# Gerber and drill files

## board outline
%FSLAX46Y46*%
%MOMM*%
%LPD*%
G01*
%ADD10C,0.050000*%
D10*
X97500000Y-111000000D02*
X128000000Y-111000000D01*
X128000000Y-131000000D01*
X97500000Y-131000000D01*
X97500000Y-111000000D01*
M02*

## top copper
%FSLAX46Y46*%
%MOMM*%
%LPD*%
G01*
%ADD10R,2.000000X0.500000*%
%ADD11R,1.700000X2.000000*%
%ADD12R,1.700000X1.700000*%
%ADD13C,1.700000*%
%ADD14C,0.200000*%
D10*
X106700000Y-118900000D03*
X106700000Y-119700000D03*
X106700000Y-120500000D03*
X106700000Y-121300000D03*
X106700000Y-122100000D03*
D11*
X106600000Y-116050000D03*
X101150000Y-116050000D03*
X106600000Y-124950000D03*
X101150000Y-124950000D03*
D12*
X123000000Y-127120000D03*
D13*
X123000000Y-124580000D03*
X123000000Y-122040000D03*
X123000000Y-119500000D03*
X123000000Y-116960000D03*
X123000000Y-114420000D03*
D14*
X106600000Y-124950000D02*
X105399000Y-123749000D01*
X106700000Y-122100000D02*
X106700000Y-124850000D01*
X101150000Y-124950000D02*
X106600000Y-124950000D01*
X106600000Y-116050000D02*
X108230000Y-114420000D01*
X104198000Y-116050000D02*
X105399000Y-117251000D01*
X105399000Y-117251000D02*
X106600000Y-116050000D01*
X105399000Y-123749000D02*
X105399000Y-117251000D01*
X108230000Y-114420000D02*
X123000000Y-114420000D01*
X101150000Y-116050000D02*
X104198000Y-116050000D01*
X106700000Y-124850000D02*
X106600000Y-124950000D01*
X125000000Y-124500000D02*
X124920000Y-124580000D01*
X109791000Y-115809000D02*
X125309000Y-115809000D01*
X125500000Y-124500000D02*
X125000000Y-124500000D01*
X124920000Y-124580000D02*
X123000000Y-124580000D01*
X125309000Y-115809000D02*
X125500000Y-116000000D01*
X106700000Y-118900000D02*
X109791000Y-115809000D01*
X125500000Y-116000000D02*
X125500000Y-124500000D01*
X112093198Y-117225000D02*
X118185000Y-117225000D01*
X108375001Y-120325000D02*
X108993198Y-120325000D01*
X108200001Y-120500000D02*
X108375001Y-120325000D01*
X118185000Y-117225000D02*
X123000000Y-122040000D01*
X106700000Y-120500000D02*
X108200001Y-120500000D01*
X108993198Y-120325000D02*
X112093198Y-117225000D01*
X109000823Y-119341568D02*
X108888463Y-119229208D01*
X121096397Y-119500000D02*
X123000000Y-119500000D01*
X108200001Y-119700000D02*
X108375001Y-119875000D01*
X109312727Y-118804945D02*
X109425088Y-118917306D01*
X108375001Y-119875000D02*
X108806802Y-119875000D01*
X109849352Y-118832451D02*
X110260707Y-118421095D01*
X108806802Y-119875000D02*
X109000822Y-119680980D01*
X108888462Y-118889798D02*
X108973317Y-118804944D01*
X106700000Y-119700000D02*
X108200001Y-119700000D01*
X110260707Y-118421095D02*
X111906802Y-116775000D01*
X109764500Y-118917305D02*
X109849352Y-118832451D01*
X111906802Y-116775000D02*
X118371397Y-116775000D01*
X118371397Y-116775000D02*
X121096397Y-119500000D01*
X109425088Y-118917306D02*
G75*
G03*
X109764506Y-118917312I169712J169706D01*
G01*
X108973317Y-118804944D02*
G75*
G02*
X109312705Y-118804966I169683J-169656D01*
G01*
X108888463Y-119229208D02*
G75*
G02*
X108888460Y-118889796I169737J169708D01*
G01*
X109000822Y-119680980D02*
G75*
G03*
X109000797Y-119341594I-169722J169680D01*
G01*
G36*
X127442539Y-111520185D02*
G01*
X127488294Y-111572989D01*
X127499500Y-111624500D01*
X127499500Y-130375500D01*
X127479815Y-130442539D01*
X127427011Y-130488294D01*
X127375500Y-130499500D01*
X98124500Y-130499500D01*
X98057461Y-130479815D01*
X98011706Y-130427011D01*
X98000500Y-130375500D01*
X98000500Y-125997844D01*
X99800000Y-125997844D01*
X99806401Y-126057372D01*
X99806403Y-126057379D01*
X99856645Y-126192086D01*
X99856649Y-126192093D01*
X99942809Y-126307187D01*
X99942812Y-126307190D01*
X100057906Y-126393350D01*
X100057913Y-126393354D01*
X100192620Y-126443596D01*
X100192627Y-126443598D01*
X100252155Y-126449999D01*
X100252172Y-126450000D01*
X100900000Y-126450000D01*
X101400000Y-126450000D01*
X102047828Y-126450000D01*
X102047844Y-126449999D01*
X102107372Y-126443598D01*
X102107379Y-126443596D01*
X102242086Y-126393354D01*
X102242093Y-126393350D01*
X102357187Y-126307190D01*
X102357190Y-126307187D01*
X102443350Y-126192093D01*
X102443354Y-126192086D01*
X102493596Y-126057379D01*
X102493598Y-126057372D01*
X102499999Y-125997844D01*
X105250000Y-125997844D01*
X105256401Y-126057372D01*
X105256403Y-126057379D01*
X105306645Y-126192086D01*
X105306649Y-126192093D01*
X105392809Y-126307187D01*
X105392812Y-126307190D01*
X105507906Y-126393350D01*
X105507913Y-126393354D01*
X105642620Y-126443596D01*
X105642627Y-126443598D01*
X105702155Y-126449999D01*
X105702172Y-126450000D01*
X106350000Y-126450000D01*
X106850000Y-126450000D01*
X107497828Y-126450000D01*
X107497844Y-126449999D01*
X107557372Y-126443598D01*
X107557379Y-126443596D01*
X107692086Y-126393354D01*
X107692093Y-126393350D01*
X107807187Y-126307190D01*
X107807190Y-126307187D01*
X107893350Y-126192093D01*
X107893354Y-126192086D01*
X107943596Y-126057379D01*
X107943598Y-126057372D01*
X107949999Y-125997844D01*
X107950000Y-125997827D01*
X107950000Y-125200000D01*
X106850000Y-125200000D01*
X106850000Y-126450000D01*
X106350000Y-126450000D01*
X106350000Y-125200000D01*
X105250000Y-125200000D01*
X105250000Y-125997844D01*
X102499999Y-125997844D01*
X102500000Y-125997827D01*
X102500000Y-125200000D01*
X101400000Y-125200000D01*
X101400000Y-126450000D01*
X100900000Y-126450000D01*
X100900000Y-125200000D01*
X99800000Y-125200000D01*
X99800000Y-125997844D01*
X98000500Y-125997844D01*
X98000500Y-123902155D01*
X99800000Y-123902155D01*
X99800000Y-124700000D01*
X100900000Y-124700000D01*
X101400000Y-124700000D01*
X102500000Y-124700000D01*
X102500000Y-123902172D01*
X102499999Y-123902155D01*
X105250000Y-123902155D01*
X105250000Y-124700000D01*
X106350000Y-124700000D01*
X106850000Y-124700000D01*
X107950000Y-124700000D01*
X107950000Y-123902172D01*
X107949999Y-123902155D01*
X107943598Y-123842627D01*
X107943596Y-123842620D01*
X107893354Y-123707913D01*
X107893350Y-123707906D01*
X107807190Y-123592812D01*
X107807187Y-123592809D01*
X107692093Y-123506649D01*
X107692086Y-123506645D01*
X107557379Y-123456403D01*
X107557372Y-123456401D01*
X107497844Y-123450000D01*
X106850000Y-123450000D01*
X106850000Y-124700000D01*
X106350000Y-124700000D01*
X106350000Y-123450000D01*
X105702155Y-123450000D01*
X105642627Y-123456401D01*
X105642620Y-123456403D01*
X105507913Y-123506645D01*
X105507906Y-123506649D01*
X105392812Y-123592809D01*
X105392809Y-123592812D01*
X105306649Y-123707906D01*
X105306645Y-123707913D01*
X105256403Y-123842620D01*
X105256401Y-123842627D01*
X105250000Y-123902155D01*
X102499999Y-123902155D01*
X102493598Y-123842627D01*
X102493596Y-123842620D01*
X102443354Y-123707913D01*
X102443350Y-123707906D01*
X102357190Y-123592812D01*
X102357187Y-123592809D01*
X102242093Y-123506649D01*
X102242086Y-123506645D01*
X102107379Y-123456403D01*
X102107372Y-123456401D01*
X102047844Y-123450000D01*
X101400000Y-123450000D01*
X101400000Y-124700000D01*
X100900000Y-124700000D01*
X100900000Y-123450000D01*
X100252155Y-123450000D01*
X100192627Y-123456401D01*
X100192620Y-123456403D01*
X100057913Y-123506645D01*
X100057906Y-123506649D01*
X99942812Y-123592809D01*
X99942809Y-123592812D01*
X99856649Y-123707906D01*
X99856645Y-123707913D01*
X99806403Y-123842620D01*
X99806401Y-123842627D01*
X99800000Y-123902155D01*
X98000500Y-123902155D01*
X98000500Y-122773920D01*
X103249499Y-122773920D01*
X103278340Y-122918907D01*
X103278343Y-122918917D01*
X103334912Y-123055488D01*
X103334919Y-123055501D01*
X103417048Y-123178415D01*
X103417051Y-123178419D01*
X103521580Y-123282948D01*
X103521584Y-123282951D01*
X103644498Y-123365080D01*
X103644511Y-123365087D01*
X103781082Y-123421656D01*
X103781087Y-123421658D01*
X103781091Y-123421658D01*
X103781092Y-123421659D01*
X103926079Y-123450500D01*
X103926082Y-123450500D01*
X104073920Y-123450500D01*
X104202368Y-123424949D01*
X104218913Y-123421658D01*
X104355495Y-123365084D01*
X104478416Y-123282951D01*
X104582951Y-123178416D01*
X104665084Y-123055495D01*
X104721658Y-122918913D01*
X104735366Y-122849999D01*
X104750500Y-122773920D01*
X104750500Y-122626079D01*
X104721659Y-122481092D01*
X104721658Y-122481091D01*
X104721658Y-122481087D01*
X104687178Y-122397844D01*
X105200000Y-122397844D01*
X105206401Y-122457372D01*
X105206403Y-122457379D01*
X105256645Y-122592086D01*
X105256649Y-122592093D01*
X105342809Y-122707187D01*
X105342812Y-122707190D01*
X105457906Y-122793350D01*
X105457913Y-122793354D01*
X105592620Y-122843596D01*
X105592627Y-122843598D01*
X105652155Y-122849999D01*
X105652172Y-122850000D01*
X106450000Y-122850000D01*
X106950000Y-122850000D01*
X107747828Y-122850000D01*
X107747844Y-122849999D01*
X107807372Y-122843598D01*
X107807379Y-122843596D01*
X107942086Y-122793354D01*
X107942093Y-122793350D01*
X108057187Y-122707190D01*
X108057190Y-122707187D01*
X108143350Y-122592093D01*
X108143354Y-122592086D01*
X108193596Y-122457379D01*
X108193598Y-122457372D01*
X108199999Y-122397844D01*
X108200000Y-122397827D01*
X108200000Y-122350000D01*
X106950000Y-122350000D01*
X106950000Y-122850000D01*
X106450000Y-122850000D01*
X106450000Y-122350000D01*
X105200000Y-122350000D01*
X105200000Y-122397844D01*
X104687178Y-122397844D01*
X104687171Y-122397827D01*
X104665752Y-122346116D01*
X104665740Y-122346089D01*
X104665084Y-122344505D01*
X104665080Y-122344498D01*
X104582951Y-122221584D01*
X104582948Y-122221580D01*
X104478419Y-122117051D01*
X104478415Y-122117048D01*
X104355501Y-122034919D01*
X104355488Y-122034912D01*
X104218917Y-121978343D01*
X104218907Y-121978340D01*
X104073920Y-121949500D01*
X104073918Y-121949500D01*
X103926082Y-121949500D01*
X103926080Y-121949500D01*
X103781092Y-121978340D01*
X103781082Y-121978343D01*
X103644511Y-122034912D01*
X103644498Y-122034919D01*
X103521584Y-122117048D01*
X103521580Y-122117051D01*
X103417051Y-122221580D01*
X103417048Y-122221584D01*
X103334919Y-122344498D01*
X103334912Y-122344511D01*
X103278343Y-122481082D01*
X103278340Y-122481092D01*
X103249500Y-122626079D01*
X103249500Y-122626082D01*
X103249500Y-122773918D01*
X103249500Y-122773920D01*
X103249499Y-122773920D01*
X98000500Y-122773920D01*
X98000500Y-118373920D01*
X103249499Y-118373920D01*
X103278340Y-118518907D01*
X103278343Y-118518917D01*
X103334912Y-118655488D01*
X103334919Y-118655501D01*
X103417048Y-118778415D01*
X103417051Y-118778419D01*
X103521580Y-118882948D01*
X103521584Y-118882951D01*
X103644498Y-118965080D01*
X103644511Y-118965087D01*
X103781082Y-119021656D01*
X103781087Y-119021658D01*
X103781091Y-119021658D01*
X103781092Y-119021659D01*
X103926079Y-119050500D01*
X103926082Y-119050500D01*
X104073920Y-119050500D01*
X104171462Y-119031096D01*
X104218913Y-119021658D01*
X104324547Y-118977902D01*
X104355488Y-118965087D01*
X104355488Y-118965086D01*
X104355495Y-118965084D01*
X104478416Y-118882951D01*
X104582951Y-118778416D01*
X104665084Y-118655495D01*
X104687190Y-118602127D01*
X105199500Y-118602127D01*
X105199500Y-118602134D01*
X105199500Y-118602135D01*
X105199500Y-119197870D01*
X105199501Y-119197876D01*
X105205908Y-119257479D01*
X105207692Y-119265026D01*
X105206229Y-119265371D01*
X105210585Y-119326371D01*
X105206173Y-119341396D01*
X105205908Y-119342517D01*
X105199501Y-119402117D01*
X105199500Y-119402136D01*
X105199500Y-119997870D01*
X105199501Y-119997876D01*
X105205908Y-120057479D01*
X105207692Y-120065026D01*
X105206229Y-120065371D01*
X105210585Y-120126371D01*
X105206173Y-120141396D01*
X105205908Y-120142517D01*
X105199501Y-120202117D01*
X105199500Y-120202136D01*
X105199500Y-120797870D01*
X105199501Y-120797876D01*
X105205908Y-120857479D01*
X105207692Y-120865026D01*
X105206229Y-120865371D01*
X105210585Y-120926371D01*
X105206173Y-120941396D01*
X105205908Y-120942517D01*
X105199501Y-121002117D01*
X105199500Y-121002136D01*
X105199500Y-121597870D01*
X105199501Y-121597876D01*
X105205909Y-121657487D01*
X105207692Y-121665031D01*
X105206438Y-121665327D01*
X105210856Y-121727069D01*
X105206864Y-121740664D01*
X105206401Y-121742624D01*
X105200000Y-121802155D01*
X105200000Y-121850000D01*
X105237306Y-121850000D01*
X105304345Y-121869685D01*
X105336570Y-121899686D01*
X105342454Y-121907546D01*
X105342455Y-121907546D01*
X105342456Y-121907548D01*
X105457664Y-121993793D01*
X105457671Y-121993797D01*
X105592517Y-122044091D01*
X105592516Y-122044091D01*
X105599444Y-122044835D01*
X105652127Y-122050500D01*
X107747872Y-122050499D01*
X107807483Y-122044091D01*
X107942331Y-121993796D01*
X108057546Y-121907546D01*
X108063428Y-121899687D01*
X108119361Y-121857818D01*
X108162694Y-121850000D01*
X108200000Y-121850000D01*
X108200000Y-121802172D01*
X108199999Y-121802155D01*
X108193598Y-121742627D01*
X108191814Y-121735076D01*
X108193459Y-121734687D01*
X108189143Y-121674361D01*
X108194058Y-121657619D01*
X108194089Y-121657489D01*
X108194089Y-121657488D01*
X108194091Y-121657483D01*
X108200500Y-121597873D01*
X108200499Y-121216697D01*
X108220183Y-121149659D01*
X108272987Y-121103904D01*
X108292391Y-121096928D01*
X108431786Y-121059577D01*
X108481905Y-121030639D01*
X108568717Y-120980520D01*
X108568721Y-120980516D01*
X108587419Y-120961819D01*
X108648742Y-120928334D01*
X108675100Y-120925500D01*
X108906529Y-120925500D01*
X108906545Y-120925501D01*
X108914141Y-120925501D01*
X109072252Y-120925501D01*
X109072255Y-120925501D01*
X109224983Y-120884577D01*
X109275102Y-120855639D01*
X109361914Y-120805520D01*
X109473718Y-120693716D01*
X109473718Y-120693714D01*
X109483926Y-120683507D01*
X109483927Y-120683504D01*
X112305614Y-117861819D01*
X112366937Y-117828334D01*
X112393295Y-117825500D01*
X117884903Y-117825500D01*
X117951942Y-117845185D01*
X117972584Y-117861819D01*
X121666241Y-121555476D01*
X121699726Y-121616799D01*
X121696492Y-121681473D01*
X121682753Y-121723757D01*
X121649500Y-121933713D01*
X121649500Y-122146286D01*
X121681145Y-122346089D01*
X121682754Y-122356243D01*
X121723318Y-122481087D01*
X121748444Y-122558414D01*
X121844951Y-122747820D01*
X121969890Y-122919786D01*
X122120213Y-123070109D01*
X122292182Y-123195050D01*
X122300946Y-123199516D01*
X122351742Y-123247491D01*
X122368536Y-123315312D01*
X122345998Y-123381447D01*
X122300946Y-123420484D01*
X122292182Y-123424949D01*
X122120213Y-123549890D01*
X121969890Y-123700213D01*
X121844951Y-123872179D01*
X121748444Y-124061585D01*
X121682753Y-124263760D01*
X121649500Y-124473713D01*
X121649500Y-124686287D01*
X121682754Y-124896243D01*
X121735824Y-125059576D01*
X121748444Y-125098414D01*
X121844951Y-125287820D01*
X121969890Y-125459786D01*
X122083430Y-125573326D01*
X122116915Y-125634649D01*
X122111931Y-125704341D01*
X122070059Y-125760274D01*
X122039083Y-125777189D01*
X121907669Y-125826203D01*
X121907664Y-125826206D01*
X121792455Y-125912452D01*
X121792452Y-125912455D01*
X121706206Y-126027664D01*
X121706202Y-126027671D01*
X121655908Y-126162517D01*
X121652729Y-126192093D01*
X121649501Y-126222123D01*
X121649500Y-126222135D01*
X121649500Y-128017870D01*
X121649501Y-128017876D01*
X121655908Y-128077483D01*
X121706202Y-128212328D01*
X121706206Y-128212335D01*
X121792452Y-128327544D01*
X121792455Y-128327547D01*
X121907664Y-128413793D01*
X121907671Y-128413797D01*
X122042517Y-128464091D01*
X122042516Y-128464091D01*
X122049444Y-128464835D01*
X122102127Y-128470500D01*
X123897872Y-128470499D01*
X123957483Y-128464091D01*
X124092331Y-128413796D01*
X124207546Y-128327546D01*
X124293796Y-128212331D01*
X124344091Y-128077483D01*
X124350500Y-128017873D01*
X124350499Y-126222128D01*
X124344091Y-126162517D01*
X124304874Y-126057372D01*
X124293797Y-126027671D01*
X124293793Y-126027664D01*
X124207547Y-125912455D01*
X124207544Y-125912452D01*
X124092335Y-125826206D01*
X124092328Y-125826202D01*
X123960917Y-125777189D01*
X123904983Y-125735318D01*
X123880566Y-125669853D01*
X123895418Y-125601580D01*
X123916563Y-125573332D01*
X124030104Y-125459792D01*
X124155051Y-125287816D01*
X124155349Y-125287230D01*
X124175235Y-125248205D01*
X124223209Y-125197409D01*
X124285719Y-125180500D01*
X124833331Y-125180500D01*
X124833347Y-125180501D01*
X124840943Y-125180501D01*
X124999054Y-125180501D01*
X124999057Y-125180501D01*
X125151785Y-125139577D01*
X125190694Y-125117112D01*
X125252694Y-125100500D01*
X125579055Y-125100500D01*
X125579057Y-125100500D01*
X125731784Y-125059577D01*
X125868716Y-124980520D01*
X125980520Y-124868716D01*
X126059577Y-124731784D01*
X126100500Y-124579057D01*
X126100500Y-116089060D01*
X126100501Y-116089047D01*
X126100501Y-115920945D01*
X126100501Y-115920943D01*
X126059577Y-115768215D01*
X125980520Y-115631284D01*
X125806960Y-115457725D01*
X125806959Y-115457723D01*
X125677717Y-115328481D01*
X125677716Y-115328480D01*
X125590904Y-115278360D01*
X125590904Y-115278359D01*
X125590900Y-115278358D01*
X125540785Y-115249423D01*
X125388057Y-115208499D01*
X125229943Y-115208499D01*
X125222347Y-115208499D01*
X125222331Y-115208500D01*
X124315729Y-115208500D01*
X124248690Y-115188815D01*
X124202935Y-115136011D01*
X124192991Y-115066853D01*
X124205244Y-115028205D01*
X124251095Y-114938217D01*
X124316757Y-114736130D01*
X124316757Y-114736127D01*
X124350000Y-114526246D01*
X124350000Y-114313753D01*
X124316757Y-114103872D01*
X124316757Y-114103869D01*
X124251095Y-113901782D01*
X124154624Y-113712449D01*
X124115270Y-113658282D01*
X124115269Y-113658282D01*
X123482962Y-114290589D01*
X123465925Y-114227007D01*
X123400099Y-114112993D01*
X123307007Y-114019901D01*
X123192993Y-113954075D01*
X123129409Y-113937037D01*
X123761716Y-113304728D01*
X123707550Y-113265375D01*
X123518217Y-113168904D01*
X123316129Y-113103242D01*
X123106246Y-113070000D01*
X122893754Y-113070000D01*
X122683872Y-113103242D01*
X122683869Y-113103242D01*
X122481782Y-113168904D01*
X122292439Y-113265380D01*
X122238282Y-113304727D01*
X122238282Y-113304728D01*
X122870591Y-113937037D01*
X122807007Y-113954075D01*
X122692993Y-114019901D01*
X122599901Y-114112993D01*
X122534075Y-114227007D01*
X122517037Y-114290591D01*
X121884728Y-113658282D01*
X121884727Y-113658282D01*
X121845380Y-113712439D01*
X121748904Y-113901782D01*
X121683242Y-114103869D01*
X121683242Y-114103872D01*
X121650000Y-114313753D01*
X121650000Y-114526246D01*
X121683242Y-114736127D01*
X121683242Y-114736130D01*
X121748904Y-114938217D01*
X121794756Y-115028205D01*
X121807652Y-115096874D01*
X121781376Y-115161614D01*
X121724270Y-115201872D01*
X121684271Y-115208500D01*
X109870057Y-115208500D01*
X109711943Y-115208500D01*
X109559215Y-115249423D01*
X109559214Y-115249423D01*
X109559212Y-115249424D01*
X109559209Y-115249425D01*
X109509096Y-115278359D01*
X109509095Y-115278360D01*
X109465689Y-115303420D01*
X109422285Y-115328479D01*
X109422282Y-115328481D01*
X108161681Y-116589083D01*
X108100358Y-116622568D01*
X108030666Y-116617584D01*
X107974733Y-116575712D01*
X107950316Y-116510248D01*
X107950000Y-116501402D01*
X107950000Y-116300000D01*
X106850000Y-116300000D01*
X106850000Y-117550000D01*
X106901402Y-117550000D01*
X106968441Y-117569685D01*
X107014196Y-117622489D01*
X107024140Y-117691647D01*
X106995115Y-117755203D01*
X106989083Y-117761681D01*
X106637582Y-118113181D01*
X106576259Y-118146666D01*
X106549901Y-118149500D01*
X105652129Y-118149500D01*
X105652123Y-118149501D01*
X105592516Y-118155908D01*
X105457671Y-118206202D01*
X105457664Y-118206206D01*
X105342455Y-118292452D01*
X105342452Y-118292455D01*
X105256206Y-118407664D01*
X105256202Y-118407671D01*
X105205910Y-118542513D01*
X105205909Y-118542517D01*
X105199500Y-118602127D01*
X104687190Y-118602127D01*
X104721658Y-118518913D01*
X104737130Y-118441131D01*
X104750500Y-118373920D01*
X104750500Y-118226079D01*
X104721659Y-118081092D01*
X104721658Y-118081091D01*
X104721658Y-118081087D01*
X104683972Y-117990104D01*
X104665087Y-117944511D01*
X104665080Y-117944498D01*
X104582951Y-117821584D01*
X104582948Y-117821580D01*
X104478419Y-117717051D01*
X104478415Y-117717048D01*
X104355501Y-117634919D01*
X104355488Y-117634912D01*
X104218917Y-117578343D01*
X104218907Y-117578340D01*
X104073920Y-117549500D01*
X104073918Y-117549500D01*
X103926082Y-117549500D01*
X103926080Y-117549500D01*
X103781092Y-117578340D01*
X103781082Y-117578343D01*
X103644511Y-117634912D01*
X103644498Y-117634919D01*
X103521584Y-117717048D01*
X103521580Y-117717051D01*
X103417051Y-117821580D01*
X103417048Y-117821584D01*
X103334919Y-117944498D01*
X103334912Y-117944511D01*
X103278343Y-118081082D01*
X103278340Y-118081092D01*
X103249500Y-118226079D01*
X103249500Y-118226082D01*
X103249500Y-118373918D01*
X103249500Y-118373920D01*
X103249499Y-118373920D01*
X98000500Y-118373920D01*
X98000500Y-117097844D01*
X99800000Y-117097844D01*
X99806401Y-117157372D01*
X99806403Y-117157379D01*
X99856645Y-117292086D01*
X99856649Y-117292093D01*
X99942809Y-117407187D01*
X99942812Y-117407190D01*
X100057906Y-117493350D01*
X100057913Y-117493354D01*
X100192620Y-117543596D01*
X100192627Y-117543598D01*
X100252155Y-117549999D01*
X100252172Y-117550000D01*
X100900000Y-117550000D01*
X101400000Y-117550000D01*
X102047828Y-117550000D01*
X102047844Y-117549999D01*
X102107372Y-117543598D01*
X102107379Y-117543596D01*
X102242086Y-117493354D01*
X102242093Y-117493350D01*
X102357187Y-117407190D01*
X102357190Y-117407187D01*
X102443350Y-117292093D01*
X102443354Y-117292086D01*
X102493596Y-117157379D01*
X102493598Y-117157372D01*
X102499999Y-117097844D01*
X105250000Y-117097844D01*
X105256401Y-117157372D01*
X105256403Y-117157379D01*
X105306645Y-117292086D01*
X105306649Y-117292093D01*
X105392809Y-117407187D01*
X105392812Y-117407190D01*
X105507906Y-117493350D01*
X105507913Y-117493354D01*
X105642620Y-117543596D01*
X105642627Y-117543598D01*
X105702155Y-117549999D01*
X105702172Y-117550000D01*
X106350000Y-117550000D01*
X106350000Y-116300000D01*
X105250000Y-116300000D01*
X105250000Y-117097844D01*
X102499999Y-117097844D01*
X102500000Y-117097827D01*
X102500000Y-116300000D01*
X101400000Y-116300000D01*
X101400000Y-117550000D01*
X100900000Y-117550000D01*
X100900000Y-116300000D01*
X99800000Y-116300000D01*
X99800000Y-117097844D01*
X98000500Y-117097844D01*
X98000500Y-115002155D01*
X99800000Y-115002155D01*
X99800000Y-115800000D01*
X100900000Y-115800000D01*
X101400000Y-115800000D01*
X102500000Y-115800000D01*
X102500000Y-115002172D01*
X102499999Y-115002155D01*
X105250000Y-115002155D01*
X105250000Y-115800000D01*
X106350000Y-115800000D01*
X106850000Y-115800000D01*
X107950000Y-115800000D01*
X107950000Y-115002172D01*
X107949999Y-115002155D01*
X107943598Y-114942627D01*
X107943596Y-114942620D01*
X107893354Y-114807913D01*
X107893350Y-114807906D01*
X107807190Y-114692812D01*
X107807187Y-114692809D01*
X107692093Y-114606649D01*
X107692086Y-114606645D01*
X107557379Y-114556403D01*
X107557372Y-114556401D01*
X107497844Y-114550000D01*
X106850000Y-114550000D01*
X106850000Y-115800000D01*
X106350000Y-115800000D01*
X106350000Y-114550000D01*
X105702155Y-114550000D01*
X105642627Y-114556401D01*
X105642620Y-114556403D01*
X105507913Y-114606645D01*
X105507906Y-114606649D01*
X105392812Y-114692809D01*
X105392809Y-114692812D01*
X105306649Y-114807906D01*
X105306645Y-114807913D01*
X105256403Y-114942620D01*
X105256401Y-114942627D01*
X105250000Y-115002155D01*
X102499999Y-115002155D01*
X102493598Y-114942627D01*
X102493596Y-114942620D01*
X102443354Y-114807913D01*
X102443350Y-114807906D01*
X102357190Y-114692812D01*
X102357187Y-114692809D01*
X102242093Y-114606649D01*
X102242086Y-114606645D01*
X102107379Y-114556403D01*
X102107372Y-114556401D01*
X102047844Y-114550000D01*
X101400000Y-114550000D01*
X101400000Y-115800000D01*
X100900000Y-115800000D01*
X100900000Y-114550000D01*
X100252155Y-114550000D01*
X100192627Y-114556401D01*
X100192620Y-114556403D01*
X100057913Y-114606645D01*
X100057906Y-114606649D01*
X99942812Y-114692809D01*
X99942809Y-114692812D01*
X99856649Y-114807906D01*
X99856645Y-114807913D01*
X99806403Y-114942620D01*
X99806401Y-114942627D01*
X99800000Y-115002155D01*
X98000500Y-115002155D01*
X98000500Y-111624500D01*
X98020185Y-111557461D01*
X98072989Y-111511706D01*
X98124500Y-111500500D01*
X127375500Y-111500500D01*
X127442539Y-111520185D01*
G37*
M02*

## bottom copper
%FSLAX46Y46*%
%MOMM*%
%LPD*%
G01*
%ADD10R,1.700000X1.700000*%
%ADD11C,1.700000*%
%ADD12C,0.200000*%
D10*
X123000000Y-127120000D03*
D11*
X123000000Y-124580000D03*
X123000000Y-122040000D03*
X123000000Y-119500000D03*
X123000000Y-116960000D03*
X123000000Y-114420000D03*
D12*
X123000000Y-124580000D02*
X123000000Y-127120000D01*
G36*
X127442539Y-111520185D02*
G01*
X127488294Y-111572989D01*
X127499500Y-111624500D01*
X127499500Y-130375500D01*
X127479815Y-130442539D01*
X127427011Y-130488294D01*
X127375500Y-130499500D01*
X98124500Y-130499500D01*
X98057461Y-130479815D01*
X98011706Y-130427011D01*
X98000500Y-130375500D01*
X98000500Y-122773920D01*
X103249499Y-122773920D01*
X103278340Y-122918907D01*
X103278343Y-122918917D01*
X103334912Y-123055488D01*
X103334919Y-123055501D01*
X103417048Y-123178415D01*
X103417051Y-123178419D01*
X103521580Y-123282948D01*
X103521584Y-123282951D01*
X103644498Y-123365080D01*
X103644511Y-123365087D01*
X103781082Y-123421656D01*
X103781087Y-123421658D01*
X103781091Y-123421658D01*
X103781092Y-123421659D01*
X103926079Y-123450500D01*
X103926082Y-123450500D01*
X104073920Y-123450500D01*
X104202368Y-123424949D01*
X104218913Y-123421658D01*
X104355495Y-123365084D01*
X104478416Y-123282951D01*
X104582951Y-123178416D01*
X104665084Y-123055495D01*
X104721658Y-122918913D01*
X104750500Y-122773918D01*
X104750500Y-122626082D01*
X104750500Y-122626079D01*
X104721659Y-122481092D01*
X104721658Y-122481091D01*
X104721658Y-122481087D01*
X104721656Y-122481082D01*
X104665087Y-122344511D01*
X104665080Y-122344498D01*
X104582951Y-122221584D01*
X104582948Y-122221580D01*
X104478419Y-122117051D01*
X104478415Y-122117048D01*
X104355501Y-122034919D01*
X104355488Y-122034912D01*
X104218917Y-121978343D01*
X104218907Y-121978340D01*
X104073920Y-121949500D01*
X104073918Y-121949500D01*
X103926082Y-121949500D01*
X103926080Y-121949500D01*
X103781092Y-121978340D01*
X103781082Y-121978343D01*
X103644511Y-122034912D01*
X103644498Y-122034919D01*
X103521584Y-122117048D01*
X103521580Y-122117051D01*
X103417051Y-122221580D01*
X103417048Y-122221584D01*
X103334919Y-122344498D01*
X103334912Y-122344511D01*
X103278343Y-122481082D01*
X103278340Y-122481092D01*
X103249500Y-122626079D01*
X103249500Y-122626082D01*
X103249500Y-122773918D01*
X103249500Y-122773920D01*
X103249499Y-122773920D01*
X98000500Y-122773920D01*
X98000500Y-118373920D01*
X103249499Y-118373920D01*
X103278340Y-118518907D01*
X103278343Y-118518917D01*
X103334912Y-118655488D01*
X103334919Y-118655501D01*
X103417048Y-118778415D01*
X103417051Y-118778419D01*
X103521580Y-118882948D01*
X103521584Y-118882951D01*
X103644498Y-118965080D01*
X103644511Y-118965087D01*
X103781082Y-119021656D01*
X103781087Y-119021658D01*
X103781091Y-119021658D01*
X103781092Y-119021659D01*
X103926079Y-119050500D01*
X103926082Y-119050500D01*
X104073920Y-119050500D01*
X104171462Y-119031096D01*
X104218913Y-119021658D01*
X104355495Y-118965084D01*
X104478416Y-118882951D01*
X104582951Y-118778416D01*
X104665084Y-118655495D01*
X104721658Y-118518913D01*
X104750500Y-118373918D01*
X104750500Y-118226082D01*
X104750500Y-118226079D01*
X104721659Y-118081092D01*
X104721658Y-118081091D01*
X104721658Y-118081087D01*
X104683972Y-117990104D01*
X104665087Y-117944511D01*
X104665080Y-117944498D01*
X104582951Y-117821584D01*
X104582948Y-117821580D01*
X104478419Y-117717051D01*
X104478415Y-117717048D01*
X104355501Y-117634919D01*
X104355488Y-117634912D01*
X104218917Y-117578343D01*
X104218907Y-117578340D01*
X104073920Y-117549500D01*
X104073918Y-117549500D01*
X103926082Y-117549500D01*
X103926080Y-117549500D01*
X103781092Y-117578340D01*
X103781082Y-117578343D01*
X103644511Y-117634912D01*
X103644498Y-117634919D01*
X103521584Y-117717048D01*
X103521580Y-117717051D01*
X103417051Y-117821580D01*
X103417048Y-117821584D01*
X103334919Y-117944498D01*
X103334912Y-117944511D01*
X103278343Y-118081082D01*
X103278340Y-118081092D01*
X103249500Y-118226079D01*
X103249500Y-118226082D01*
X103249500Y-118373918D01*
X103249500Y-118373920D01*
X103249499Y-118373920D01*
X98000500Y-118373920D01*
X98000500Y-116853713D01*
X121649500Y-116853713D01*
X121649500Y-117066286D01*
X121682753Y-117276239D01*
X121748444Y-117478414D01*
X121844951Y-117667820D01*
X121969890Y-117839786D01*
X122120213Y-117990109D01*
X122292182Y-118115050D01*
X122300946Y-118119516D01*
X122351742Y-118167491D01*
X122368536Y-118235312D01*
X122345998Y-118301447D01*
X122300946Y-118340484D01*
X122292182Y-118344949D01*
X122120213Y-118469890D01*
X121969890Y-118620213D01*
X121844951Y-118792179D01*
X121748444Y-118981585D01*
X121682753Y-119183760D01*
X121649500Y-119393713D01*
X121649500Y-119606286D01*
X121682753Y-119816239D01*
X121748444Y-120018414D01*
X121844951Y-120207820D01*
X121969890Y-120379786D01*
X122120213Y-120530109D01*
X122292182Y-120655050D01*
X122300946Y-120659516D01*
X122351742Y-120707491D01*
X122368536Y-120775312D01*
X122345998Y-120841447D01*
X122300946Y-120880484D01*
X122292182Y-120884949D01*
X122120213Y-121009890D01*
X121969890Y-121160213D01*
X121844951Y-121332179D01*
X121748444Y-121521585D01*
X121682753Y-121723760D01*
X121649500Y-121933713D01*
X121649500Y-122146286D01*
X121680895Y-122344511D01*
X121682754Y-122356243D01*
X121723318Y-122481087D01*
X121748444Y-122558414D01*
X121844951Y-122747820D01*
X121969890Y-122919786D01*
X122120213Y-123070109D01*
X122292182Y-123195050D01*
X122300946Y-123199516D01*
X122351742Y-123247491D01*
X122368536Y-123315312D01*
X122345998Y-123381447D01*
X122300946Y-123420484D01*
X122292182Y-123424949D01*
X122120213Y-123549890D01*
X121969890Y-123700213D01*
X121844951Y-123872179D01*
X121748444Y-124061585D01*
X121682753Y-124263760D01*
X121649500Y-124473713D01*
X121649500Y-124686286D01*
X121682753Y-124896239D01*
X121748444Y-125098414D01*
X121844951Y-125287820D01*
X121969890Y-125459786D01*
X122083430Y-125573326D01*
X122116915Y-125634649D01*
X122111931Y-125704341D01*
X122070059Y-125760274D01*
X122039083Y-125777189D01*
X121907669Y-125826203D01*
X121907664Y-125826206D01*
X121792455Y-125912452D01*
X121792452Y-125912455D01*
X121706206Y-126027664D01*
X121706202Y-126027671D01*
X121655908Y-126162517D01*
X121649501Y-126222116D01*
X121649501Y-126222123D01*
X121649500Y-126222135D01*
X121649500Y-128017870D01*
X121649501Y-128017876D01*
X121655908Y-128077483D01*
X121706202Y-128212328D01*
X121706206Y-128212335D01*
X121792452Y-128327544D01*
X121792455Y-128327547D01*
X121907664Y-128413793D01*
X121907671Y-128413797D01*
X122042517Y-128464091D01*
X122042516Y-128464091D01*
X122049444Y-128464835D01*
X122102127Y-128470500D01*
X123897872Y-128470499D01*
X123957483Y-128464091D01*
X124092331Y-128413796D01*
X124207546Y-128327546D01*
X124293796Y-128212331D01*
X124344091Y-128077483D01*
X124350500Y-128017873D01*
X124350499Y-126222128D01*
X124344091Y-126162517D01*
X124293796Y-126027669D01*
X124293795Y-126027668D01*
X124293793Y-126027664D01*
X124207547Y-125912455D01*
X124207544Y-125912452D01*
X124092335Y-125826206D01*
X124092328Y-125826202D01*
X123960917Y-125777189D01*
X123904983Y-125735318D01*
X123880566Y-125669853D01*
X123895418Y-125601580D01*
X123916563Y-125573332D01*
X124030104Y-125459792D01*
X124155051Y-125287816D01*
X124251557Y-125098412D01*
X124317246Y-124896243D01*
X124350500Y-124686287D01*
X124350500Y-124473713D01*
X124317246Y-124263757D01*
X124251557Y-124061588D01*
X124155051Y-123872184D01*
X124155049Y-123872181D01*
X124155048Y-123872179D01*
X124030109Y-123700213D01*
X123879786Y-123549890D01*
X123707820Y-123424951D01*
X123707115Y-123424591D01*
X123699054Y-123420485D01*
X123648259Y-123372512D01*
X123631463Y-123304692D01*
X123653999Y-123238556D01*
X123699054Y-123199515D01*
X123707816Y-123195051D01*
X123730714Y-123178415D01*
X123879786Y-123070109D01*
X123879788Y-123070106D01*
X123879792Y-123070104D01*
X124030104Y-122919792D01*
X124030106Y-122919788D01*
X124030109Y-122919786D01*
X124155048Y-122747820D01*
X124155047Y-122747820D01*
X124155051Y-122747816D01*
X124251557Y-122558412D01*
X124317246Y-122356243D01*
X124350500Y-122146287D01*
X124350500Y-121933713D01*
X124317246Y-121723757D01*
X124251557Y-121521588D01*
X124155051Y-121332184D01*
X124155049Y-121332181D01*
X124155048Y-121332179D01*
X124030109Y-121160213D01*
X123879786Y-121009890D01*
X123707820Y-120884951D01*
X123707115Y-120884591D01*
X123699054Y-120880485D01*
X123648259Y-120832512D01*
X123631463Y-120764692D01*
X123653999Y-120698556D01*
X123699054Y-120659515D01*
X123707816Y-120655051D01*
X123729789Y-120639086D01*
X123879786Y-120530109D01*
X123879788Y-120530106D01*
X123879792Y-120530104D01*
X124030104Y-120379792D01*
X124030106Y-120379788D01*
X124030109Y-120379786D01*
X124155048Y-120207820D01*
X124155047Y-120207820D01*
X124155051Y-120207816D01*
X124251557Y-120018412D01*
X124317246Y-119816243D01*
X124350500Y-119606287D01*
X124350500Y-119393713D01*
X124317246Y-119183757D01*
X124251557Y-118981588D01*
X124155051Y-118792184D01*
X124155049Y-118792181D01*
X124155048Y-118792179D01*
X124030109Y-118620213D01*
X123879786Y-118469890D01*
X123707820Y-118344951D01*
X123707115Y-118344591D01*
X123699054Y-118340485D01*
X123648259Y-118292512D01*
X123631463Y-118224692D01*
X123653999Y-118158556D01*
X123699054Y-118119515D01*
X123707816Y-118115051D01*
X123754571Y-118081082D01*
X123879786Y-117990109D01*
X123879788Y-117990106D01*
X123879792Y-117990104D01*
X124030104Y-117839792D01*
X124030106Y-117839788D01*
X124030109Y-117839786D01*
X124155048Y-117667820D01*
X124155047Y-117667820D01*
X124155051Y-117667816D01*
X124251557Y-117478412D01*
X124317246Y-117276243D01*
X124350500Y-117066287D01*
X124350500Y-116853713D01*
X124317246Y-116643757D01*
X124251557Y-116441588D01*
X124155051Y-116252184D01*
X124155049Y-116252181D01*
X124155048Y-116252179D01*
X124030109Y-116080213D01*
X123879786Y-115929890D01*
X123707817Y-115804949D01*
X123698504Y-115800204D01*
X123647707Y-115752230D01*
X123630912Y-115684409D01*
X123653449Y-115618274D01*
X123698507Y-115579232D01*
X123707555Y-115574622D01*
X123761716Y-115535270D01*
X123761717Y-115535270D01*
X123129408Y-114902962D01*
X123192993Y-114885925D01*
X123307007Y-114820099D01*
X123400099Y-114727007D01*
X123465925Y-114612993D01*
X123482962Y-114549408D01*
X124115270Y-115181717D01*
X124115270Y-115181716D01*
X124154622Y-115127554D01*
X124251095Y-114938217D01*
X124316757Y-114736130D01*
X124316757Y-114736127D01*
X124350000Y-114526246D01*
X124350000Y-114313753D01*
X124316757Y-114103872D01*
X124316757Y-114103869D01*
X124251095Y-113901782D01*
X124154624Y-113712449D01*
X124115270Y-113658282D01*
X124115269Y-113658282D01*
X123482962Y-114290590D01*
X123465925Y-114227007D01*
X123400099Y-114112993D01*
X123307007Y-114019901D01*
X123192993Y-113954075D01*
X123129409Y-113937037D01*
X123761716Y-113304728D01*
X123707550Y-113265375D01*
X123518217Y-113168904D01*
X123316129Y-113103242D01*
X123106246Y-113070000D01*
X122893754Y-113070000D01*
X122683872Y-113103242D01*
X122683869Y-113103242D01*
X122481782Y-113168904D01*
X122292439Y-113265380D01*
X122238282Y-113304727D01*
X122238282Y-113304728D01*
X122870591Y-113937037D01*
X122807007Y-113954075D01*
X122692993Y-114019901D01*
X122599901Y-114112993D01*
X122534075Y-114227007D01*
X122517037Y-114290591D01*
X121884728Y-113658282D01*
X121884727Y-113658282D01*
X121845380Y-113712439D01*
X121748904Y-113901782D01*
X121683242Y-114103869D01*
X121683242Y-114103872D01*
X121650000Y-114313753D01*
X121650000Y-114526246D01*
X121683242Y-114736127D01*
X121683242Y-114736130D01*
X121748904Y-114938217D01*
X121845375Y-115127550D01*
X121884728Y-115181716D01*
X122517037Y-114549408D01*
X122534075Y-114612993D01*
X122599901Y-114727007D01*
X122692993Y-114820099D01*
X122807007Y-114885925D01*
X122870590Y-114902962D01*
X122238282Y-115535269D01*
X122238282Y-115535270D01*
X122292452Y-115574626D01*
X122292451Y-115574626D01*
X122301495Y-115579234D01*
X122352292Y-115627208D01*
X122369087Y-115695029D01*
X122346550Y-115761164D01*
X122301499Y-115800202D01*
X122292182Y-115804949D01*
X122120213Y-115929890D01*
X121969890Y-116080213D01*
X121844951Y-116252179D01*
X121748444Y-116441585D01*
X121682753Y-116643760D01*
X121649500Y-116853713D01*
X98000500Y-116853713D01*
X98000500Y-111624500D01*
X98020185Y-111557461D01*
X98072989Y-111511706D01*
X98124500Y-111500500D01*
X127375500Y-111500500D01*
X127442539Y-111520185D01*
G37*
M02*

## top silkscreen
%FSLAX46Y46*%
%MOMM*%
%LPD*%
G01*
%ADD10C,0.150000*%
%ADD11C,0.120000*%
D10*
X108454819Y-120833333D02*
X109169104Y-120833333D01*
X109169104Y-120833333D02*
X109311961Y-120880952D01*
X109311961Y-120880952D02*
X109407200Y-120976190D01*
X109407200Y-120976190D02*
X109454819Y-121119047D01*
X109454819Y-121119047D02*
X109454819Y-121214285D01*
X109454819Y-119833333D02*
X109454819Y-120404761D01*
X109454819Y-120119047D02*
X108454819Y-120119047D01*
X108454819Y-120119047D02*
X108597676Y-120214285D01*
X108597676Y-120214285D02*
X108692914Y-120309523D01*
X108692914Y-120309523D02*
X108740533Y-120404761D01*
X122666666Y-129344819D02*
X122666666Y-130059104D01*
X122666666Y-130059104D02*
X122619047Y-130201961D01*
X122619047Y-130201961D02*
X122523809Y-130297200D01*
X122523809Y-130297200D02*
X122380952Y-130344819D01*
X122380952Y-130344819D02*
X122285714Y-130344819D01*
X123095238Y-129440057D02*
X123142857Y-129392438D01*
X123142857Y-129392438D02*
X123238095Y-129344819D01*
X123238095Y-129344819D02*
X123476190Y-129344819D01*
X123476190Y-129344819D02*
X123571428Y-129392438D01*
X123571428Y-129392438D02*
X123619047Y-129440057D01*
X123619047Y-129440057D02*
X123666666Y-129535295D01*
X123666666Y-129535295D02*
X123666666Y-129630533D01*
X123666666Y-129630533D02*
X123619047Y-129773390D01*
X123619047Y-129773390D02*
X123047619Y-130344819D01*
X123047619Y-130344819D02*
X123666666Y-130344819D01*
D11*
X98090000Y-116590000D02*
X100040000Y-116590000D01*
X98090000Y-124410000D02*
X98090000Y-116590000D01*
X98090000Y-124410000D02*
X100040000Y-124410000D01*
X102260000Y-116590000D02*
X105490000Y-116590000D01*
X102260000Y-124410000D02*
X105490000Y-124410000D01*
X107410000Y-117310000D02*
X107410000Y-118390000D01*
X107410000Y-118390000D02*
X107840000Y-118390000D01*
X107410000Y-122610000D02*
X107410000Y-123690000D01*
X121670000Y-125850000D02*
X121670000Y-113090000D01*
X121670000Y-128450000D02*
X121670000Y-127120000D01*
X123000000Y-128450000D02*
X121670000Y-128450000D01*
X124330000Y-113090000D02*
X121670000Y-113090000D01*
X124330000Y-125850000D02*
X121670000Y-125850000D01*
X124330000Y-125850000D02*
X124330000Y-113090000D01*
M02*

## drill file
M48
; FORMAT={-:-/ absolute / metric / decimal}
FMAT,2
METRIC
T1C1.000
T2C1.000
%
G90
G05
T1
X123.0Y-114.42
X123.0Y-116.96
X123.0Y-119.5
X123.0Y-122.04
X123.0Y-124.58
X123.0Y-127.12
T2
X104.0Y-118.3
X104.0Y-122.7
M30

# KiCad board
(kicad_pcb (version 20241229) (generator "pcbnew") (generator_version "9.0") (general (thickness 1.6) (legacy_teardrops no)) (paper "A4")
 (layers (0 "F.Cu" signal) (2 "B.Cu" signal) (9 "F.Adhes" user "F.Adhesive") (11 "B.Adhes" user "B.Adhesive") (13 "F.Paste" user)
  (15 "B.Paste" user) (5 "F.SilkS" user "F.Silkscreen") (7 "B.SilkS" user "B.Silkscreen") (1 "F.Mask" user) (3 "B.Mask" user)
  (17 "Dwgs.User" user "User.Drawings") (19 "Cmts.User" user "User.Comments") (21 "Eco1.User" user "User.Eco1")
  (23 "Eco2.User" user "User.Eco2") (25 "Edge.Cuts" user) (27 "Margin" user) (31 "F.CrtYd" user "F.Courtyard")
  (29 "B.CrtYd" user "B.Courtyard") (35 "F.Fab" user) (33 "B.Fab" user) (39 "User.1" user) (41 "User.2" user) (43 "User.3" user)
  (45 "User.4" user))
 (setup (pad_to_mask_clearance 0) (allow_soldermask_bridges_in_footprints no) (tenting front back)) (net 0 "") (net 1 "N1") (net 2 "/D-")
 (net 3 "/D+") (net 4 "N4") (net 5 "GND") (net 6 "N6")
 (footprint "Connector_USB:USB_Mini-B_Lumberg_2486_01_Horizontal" (layer "F.Cu") (at 104 120.5 -90)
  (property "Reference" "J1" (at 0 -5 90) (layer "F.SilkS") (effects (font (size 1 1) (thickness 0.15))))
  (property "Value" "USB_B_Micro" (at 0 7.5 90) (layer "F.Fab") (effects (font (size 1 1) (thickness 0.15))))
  (fp_line (start -3.91 5.91) (end -3.91 3.96) (stroke (width 0.12) (type solid)) (layer "F.SilkS"))
  (fp_line (start 3.91 5.91) (end -3.91 5.91) (stroke (width 0.12) (type solid)) (layer "F.SilkS"))
  (fp_line (start 3.91 5.91) (end 3.91 3.96) (stroke (width 0.12) (type solid)) (layer "F.SilkS"))
  (fp_line (start -3.91 1.74) (end -3.91 -1.49) (stroke (width 0.12) (type solid)) (layer "F.SilkS"))
  (fp_line (start 3.91 1.74) (end 3.91 -1.49) (stroke (width 0.12) (type solid)) (layer "F.SilkS"))
  (fp_line (start -3.19 -3.41) (end -2.11 -3.41) (stroke (width 0.12) (type solid)) (layer "F.SilkS"))
  (fp_line (start -2.11 -3.41) (end -2.11 -3.84) (stroke (width 0.12) (type solid)) (layer "F.SilkS"))
  (fp_line (start 2.11 -3.41) (end 3.19 -3.41) (stroke (width 0.12) (type solid)) (layer "F.SilkS"))
  (pad "" np_thru_hole circle (at -2.2 0 270) (size 1 1) (drill 1) (layers "*.Cu" "*.Mask"))
  (pad "" np_thru_hole circle (at 2.2 0 270) (size 1 1) (drill 1) (layers "*.Cu" "*.Mask"))
  (pad "1" smd rect (at -1.6 -2.7 270) (size 0.5 2) (layers "F.Cu" "F.Mask" "F.Paste") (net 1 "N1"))
  (pad "2" smd rect (at -0.8 -2.7 270) (size 0.5 2) (layers "F.Cu" "F.Mask" "F.Paste") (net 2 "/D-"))
  (pad "3" smd rect (at 0 -2.7 270) (size 0.5 2) (layers "F.Cu" "F.Mask" "F.Paste") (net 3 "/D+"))
  (pad "4" smd rect (at 0.8 -2.7 270) (size 0.5 2) (layers "F.Cu" "F.Mask" "F.Paste") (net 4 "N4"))
  (pad "5" smd rect (at 1.6 -2.7 270) (size 0.5 2) (layers "F.Cu" "F.Mask" "F.Paste") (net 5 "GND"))
  (pad "6" smd rect (at -4.45 -2.6 270) (size 2 1.7) (layers "F.Cu" "F.Mask" "F.Paste") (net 5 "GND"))
  (pad "6" smd rect (at -4.45 2.85 270) (size 2 1.7) (layers "F.Cu" "F.Mask" "F.Paste") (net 5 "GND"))
  (pad "6" smd rect (at 4.45 -2.6 270) (size 2 1.7) (layers "F.Cu" "F.Mask" "F.Paste") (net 5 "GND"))
  (pad "6" smd rect (at 4.45 2.85 270) (size 2 1.7) (layers "F.Cu" "F.Mask" "F.Paste") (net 5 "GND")))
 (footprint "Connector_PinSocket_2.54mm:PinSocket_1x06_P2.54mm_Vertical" (layer "F.Cu") (at 123 127.12 180)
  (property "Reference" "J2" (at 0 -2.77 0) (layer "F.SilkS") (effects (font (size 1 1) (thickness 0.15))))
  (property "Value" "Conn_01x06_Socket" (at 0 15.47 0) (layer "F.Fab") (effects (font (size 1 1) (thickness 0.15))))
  (fp_line (start 1.33 1.27) (end 1.33 14.03) (stroke (width 0.12) (type solid)) (layer "F.SilkS"))
  (fp_line (start 1.33 -1.33) (end 1.33 0) (stroke (width 0.12) (type solid)) (layer "F.SilkS"))
  (fp_line (start 0 -1.33) (end 1.33 -1.33) (stroke (width 0.12) (type solid)) (layer "F.SilkS"))
  (fp_line (start -1.33 14.03) (end 1.33 14.03) (stroke (width 0.12) (type solid)) (layer "F.SilkS"))
  (fp_line (start -1.33 1.27) (end 1.33 1.27) (stroke (width 0.12) (type solid)) (layer "F.SilkS"))
  (fp_line (start -1.33 1.27) (end -1.33 14.03) (stroke (width 0.12) (type solid)) (layer "F.SilkS"))
  (pad "1" thru_hole rect (at 0 0 180) (size 1.7 1.7) (drill 1) (layers "*.Cu" "*.Mask") (remove_unused_layers no) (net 1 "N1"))
  (pad "2" thru_hole circle (at 0 2.54 180) (size 1.7 1.7) (drill 1) (layers "*.Cu" "*.Mask") (remove_unused_layers no) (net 1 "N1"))
  (pad "3" thru_hole circle (at 0 5.08 180) (size 1.7 1.7) (drill 1) (layers "*.Cu" "*.Mask") (remove_unused_layers no) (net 3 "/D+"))
  (pad "4" thru_hole circle (at 0 7.62 180) (size 1.7 1.7) (drill 1) (layers "*.Cu" "*.Mask") (remove_unused_layers no) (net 2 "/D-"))
  (pad "5" thru_hole circle (at 0 10.16 180) (size 1.7 1.7) (drill 1) (layers "*.Cu" "*.Mask") (remove_unused_layers no) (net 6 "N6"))
  (pad "6" thru_hole circle (at 0 12.7 180) (size 1.7 1.7) (drill 1) (layers "*.Cu" "*.Mask") (remove_unused_layers no) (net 5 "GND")))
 (gr_rect (start 97.5 111) (end 128 131) (stroke (width 0.05) (type default)) (fill no) (layer "Edge.Cuts"))
 (segment (start 106.6 124.95) (end 105.399 123.749) (width 0.2) (layer "F.Cu") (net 5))
 (segment (start 106.7 122.1) (end 106.7 124.85) (width 0.2) (layer "F.Cu") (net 5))
 (segment (start 101.15 124.95) (end 106.6 124.95) (width 0.2) (layer "F.Cu") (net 5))
 (segment (start 106.6 116.05) (end 108.23 114.42) (width 0.2) (layer "F.Cu") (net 5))
 (segment (start 104.198 116.05) (end 105.399 117.251) (width 0.2) (layer "F.Cu") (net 5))
 (segment (start 105.399 117.251) (end 106.6 116.05) (width 0.2) (layer "F.Cu") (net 5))
 (segment (start 105.399 123.749) (end 105.399 117.251) (width 0.2) (layer "F.Cu") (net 5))
 (segment (start 108.23 114.42) (end 123 114.42) (width 0.2) (layer "F.Cu") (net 5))
 (segment (start 101.15 116.05) (end 104.198 116.05) (width 0.2) (layer "F.Cu") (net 5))
 (segment (start 106.7 124.85) (end 106.6 124.95) (width 0.2) (layer "F.Cu") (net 5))
 (segment (start 125 124.5) (end 124.92 124.58) (width 0.2) (layer "F.Cu") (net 1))
 (segment (start 109.791 115.809) (end 125.309 115.809) (width 0.2) (layer "F.Cu") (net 1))
 (segment (start 125.5 124.5) (end 125 124.5) (width 0.2) (layer "F.Cu") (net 1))
 (segment (start 124.92 124.58) (end 123 124.58) (width 0.2) (layer "F.Cu") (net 1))
 (segment (start 125.309 115.809) (end 125.5 116) (width 0.2) (layer "F.Cu") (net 1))
 (segment (start 106.7 118.9) (end 109.791 115.809) (width 0.2) (layer "F.Cu") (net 1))
 (segment (start 125.5 116) (end 125.5 124.5) (width 0.2) (layer "F.Cu") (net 1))
 (segment (start 123 124.58) (end 123 127.12) (width 0.2) (layer "B.Cu") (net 1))
 (segment (start 112.093198 117.225) (end 118.185 117.225) (width 0.2) (layer "F.Cu") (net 3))
 (segment (start 108.375001 120.325) (end 108.993198 120.325) (width 0.2) (layer "F.Cu") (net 3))
 (segment (start 108.200001 120.5) (end 108.375001 120.325) (width 0.2) (layer "F.Cu") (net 3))
 (segment (start 118.185 117.225) (end 123 122.04) (width 0.2) (layer "F.Cu") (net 3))
 (segment (start 106.7 120.5) (end 108.200001 120.5) (width 0.2) (layer "F.Cu") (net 3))
 (segment (start 108.993198 120.325) (end 112.093198 117.225) (width 0.2) (layer "F.Cu") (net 3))
 (segment (start 109.000823 119.341568) (end 108.888463 119.229208) (width 0.2) (layer "F.Cu") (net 2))
 (segment (start 121.096397 119.5) (end 123 119.5) (width 0.2) (layer "F.Cu") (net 2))
 (segment (start 108.200001 119.7) (end 108.375001 119.875) (width 0.2) (layer "F.Cu") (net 2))
 (segment (start 109.312727 118.804945) (end 109.425088 118.917306) (width 0.2) (layer "F.Cu") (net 2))
 (segment (start 108.375001 119.875) (end 108.806802 119.875) (width 0.2) (layer "F.Cu") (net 2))
 (segment (start 109.849352 118.832451) (end 110.260707 118.421095) (width 0.2) (layer "F.Cu") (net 2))
 (segment (start 108.806802 119.875) (end 109.000822 119.68098) (width 0.2) (layer "F.Cu") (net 2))
 (segment (start 108.888462 118.889798) (end 108.973317 118.804944) (width 0.2) (layer "F.Cu") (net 2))
 (segment (start 106.7 119.7) (end 108.200001 119.7) (width 0.2) (layer "F.Cu") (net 2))
 (segment (start 110.260707 118.421095) (end 111.906802 116.775) (width 0.2) (layer "F.Cu") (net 2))
 (segment (start 109.7645 118.917305) (end 109.849352 118.832451) (width 0.2) (layer "F.Cu") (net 2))
 (segment (start 111.906802 116.775) (end 118.371397 116.775) (width 0.2) (layer "F.Cu") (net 2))
 (segment (start 118.371397 116.775) (end 121.096397 119.5) (width 0.2) (layer "F.Cu") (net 2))
 (arc (start 109.425088 118.917306) (mid 109.594793 118.987601) (end 109.7645 118.917305) (width 0.2) (layer "F.Cu") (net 2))
 (arc (start 108.973317 118.804944) (mid 109.143022 118.73465) (end 109.312727 118.804945) (width 0.2) (layer "F.Cu") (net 2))
 (arc (start 108.888463 119.229208) (mid 108.818169 119.059502) (end 108.888462 118.889798) (width 0.2) (layer "F.Cu") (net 2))
 (arc (start 109.000822 119.68098) (mid 109.071117 119.511274) (end 109.000823 119.341568) (width 0.2) (layer "F.Cu") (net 2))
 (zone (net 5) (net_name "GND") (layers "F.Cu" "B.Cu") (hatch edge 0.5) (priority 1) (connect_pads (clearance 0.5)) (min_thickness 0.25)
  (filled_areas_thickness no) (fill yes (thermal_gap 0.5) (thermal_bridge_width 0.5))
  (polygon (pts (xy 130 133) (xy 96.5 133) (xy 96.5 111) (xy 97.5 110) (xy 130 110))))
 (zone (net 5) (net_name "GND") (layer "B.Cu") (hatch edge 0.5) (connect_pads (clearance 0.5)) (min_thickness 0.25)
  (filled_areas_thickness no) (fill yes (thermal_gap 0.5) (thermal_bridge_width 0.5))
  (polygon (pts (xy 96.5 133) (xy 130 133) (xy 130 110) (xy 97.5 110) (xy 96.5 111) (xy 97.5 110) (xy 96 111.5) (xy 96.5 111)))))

